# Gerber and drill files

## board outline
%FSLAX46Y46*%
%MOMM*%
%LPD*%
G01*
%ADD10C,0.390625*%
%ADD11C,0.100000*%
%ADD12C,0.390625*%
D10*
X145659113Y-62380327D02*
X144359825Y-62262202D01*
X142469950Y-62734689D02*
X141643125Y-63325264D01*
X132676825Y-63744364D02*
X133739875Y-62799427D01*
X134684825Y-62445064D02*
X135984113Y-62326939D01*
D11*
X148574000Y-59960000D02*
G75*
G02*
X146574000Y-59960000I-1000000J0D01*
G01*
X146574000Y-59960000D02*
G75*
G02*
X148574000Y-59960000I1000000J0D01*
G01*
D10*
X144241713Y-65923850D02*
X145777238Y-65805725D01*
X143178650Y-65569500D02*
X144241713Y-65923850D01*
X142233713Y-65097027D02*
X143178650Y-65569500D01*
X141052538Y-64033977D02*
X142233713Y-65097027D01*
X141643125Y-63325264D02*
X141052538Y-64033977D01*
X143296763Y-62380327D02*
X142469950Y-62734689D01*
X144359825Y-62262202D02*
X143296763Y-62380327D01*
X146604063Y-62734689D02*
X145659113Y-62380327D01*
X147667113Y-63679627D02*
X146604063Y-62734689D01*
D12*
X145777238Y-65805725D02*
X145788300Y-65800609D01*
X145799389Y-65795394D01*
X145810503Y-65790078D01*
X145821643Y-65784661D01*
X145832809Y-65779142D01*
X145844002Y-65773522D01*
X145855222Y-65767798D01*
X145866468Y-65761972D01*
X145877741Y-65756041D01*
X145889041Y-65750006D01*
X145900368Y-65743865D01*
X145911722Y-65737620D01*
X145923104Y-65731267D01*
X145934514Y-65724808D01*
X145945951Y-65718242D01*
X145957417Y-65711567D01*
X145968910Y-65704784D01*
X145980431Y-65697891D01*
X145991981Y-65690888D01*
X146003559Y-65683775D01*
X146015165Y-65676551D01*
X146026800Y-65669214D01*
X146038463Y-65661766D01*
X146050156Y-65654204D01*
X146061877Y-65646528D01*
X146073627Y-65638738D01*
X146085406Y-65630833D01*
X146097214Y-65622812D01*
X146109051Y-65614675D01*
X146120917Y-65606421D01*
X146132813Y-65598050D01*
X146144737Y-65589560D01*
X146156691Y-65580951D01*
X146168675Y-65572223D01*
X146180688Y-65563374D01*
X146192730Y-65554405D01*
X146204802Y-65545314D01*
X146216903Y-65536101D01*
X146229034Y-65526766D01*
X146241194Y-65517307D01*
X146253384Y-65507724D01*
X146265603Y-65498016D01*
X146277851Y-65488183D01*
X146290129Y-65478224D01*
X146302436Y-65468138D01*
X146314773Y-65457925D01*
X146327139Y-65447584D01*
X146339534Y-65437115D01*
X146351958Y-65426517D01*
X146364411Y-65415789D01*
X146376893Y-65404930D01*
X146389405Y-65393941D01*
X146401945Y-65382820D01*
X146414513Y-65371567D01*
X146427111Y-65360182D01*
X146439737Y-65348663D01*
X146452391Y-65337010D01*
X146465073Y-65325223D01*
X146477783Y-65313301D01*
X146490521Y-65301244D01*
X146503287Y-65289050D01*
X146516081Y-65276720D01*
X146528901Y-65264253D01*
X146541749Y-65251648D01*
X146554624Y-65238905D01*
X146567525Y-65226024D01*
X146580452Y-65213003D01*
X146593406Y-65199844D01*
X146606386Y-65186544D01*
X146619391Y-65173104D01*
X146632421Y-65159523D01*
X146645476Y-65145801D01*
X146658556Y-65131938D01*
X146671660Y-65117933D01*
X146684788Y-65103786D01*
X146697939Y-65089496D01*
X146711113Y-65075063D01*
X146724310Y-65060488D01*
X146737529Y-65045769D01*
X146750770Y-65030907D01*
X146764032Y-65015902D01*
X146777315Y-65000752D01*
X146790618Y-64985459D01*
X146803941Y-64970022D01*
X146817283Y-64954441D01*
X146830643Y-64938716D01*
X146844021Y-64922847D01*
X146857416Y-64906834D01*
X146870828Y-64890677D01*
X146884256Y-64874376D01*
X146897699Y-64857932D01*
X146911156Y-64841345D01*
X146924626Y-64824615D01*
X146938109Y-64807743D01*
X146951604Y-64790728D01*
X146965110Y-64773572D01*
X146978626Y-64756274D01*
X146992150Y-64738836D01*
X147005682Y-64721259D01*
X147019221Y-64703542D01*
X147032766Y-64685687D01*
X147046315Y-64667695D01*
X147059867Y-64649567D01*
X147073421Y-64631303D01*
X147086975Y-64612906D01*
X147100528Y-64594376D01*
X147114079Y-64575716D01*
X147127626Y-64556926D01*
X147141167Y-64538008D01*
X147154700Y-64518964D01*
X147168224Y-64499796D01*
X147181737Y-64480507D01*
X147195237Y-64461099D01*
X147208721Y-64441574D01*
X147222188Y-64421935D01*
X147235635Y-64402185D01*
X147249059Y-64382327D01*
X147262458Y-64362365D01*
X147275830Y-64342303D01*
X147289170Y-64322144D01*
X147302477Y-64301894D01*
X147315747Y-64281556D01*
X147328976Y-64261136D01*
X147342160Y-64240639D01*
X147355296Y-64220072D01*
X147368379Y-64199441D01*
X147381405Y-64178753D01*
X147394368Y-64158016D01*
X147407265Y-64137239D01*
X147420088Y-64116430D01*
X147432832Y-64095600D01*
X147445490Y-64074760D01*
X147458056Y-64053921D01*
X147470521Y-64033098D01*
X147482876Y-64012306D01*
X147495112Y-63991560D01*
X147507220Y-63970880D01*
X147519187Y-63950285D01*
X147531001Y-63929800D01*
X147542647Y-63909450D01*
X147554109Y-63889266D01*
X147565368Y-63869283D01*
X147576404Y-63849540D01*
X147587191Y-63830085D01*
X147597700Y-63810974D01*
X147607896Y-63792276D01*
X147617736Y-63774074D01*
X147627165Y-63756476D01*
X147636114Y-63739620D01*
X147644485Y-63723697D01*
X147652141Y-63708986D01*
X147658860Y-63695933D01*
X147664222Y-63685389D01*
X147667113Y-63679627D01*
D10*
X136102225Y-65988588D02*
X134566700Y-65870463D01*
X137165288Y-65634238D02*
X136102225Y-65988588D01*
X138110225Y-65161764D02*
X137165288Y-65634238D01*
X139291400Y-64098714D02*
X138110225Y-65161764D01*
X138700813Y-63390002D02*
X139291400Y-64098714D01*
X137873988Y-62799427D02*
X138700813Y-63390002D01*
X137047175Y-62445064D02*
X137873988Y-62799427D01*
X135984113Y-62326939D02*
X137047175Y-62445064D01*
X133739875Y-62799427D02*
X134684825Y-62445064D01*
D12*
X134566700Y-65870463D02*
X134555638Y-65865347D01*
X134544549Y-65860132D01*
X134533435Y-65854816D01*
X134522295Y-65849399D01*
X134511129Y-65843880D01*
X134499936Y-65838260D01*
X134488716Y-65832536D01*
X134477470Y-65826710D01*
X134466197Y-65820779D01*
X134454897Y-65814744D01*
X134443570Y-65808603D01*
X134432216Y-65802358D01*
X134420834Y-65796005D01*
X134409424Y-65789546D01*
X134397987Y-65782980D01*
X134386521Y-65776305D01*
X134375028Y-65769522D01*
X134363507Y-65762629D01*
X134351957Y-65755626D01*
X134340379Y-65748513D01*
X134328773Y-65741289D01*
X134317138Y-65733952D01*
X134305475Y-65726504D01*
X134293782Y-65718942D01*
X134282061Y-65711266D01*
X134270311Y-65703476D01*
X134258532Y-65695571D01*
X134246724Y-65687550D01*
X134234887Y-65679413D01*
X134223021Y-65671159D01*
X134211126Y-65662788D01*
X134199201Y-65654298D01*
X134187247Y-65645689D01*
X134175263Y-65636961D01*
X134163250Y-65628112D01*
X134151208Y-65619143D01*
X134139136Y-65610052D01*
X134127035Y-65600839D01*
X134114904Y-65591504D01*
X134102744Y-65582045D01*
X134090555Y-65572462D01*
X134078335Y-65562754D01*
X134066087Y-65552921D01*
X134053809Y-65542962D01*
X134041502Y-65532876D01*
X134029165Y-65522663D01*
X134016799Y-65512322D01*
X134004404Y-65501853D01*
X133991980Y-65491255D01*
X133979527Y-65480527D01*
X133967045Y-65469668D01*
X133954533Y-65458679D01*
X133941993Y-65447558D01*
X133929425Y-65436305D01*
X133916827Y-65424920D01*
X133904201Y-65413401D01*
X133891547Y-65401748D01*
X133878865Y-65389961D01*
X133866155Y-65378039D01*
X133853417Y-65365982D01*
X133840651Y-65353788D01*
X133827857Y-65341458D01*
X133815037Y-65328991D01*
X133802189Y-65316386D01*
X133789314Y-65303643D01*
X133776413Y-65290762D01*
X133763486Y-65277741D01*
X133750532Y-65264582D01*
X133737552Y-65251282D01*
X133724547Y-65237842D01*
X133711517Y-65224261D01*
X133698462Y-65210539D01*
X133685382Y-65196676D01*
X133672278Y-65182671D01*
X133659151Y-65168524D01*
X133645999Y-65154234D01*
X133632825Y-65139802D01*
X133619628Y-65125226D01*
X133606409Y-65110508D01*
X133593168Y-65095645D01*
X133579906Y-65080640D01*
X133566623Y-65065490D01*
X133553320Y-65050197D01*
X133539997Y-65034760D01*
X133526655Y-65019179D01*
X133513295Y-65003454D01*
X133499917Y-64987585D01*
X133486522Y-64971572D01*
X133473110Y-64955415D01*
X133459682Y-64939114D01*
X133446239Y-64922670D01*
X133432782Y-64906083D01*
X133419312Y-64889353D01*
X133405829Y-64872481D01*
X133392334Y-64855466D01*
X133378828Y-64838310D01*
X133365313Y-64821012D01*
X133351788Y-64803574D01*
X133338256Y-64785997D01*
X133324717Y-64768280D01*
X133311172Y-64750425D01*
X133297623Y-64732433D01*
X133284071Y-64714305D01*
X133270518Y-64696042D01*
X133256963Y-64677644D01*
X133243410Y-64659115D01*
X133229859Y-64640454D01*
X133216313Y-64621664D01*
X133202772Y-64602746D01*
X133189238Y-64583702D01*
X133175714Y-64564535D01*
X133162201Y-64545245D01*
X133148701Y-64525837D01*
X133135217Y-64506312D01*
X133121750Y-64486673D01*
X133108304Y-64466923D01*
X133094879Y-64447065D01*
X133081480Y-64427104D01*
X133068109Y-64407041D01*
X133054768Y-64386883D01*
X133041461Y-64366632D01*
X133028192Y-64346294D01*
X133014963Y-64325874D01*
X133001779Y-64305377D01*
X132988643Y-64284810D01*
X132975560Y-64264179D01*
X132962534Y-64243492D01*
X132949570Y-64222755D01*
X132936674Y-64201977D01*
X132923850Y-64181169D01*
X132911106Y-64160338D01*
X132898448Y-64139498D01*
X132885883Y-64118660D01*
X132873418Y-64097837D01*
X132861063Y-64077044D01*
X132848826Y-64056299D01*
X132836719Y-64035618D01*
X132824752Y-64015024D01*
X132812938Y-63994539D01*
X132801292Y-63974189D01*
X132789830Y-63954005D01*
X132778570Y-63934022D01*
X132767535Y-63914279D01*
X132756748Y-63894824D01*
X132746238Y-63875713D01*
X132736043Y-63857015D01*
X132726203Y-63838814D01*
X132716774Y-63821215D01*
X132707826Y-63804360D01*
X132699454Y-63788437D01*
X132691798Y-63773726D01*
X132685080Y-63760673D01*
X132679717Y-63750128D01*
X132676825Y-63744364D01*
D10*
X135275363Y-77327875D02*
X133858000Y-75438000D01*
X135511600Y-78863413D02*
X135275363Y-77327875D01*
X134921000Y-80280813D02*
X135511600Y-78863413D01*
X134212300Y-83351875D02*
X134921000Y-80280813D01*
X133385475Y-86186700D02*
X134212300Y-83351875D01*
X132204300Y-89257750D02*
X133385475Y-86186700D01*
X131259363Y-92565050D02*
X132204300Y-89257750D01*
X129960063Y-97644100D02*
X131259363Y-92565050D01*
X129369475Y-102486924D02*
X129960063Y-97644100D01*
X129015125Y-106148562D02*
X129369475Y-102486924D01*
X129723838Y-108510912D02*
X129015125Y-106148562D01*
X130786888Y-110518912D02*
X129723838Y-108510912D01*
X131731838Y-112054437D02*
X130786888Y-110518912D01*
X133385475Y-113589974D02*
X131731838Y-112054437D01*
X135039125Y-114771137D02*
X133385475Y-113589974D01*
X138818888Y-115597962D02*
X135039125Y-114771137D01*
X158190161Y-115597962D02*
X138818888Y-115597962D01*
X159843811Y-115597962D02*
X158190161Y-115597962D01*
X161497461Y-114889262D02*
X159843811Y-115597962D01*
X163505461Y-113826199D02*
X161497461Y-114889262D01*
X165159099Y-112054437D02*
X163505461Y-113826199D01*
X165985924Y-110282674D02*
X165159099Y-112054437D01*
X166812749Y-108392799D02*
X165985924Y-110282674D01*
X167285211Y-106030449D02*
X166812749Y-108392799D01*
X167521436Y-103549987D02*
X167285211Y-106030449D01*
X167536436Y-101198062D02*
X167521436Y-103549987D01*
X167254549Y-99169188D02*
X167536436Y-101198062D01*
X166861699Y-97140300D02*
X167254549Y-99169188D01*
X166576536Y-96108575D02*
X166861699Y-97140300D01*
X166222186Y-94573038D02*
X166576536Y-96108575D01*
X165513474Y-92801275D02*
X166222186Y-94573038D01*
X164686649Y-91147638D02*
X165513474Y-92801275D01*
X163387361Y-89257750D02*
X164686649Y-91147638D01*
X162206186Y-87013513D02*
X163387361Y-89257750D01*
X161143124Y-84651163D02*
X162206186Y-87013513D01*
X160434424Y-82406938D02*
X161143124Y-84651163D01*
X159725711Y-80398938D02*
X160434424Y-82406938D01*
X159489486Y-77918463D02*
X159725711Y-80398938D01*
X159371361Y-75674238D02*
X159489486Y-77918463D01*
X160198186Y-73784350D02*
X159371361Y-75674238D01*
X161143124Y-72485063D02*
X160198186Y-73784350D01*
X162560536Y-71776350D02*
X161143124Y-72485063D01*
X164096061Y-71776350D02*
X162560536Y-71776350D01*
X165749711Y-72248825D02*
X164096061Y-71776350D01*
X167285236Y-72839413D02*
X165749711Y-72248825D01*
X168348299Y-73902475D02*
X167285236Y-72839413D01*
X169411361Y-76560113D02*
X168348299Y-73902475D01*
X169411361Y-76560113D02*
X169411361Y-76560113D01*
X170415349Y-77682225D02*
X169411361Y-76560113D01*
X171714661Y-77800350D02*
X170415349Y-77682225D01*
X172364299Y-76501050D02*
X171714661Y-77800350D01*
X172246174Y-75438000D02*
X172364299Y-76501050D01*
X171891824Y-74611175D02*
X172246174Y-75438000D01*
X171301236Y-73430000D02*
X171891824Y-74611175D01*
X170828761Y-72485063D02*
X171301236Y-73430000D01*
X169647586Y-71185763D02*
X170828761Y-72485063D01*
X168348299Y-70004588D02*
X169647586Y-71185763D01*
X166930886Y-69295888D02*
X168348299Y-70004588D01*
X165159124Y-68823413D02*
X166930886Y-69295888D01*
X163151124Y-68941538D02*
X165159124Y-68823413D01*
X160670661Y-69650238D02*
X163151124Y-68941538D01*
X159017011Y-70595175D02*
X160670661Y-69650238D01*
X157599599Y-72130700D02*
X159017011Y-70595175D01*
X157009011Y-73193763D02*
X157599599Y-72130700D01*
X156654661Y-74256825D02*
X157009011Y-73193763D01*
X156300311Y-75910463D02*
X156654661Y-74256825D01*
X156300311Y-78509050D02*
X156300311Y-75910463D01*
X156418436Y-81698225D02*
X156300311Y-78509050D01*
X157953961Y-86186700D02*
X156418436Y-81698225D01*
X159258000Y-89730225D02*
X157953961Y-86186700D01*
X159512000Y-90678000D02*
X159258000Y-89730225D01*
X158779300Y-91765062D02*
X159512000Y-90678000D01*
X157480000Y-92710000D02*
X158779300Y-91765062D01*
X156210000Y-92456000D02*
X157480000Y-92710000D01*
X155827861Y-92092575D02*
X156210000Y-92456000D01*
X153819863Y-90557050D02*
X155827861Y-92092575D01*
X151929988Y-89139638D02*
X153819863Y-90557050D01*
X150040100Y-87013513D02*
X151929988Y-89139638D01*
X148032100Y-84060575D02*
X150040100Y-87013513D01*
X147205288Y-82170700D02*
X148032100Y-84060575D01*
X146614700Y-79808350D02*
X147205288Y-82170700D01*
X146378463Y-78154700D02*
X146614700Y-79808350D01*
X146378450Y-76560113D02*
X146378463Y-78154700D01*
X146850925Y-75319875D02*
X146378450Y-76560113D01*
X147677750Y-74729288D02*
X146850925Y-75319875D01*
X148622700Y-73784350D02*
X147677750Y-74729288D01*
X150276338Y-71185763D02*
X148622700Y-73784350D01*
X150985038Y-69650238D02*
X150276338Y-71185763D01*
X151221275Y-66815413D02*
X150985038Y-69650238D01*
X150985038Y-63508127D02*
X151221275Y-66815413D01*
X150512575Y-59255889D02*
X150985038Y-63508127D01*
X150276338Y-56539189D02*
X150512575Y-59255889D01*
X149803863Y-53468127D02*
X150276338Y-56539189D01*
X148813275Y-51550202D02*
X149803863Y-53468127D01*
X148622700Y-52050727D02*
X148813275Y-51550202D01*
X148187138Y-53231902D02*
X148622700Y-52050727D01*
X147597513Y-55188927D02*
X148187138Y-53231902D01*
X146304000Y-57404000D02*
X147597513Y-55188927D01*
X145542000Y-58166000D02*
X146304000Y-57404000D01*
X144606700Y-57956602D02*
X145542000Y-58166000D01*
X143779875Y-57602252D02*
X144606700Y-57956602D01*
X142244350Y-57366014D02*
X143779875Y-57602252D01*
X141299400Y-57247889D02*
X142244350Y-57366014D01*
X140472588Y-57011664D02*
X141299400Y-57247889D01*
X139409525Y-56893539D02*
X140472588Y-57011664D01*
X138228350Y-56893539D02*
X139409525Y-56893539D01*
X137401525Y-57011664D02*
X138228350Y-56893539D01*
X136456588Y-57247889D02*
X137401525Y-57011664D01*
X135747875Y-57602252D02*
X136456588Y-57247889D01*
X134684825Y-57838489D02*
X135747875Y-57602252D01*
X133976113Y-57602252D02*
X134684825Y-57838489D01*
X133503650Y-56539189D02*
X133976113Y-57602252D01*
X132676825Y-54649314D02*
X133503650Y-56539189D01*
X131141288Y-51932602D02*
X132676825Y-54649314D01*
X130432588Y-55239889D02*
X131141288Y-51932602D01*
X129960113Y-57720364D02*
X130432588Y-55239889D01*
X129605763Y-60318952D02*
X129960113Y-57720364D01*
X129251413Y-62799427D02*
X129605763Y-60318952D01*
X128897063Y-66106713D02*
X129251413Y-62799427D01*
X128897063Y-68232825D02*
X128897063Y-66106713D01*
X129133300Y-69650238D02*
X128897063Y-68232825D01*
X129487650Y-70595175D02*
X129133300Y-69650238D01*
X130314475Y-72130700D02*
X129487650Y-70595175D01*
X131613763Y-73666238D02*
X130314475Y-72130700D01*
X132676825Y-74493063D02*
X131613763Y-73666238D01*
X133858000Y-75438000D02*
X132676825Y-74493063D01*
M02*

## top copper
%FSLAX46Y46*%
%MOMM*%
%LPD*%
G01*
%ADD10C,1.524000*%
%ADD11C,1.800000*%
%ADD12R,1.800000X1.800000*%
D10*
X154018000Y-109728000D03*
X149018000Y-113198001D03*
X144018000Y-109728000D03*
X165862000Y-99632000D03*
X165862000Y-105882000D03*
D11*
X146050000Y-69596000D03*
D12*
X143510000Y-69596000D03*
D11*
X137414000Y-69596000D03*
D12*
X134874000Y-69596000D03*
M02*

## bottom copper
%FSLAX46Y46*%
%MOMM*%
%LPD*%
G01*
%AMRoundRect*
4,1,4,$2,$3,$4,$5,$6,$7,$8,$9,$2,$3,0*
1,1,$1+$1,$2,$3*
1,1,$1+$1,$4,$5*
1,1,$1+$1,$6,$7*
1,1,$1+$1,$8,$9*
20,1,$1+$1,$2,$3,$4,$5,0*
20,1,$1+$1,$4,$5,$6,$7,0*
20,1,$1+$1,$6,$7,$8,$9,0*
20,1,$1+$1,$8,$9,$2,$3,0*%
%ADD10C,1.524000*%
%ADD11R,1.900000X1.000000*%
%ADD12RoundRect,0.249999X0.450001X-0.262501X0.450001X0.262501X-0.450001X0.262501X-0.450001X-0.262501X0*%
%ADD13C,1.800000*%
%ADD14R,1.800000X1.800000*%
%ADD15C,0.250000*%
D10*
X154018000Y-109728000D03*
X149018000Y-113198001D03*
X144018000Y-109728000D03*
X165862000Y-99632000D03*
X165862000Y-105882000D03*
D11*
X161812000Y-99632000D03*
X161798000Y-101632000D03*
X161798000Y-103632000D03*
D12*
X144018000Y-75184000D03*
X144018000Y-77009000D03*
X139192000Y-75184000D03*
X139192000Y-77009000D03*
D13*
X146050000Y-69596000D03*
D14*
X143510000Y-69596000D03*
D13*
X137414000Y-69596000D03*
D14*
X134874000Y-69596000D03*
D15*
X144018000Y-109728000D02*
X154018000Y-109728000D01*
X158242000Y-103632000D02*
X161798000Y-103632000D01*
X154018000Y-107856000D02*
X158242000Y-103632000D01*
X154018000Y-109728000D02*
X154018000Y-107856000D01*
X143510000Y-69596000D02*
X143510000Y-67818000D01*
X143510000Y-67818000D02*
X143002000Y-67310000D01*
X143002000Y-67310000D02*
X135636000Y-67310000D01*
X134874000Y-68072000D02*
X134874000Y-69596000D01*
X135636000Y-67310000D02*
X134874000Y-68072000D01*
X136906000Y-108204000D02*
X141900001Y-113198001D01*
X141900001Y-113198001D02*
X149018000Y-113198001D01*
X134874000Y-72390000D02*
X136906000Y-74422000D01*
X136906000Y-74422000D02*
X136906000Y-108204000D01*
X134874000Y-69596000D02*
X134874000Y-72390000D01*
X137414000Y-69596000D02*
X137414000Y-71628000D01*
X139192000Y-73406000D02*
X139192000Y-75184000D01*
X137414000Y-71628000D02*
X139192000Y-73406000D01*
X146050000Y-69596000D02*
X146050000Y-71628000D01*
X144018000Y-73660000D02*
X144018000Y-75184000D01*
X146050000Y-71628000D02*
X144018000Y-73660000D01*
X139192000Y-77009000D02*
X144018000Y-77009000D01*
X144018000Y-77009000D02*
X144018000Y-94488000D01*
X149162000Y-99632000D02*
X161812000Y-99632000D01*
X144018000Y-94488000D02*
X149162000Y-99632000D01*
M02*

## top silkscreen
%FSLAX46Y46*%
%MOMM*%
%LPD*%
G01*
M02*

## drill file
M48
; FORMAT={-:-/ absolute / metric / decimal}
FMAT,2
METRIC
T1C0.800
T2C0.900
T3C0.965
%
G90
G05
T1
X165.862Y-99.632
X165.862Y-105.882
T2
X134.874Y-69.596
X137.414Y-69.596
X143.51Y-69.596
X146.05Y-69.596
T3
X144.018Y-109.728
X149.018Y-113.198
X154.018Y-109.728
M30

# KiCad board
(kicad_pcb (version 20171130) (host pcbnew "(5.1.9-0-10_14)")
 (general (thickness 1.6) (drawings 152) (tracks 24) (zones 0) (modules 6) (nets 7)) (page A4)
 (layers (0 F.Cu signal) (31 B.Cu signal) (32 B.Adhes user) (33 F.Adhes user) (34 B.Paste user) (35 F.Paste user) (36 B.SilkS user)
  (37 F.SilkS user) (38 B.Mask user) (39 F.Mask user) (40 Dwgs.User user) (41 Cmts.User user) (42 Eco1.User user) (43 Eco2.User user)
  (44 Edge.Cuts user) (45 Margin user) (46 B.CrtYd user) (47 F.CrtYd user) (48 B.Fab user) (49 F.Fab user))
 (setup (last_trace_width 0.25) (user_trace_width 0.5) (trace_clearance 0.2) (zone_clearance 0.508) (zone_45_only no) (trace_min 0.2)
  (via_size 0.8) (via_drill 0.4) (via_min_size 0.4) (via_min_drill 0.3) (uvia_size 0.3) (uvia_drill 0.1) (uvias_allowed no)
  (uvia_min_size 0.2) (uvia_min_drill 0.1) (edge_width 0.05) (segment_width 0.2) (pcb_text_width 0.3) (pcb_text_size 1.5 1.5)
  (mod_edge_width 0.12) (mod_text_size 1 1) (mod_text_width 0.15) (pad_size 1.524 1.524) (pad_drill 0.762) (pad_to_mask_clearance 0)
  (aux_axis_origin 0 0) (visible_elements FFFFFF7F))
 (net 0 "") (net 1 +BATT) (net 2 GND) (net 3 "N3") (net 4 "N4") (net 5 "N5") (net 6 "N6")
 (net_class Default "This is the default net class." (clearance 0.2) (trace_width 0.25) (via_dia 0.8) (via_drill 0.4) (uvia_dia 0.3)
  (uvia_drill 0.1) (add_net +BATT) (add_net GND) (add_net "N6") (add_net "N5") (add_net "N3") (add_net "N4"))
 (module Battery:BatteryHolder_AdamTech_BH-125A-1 (layer B.Cu) (at 144.018 109.728)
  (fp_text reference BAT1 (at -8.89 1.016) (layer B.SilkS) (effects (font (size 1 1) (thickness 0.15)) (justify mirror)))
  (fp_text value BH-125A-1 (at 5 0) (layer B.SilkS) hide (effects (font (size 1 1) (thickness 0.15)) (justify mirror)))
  (pad POS2 thru_hole circle (at 10 0) (size 1.524 1.524) (drill 0.9652) (layers *.Cu *.Mask) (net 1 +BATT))
  (pad NEG thru_hole circle (at 5 3.470001) (size 1.524 1.524) (drill 0.9652) (layers *.Cu *.Mask) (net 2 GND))
  (pad POS1 thru_hole circle (at 0 0) (size 1.524 1.524) (drill 0.9652) (layers *.Cu *.Mask) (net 1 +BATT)))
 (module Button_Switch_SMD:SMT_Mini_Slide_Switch (layer B.Cu) (at 163.576 102.757 270)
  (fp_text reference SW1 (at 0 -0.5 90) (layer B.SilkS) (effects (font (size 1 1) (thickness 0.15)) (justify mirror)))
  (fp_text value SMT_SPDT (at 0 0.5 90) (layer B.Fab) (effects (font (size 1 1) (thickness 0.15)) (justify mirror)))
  (pad "" thru_hole circle (at -3.125 -2.286 270) (size 1.524 1.524) (drill 0.8) (layers *.Cu *.Mask))
  (pad "" thru_hole circle (at 3.125 -2.286 270) (size 1.524 1.524) (drill 0.8) (layers *.Cu *.Mask))
  (pad 1 smd rect (at -3.125 1.764 270) (size 1 1.9) (layers B.Cu B.Paste B.Mask) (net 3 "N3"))
  (pad 2 smd rect (at -1.125 1.778 270) (size 1 1.9) (layers B.Cu B.Paste B.Mask) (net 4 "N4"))
  (pad 3 smd rect (at 0.875 1.778 270) (size 1 1.9) (layers B.Cu B.Paste B.Mask) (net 1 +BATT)))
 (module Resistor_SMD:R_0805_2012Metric (layer B.Cu) (at 144.018 76.0965 90)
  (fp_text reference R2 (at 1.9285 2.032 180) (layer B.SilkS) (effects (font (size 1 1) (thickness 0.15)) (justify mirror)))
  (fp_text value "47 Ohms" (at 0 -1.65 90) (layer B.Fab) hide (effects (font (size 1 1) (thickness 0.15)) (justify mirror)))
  (pad 2 smd roundrect (at 0.9125 0 90) (size 1.025 1.4) (layers B.Cu B.Paste B.Mask) (roundrect_rratio 0.2439014634146341) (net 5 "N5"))
  (pad 1 smd roundrect (at -0.9125 0 90) (size 1.025 1.4) (layers B.Cu B.Paste B.Mask) (roundrect_rratio 0.2439014634146341) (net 3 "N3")))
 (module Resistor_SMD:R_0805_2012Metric (layer B.Cu) (at 139.192 76.0965 90)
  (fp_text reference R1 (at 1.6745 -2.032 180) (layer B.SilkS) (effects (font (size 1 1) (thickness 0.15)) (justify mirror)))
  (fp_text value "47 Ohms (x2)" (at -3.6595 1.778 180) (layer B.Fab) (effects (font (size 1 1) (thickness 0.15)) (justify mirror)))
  (pad 2 smd roundrect (at 0.9125 0 90) (size 1.025 1.4) (layers B.Cu B.Paste B.Mask) (roundrect_rratio 0.2439014634146341) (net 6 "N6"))
  (pad 1 smd roundrect (at -0.9125 0 90) (size 1.025 1.4) (layers B.Cu B.Paste B.Mask) (roundrect_rratio 0.2439014634146341) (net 3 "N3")))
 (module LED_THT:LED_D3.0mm (layer B.Cu) (at 143.51 69.596)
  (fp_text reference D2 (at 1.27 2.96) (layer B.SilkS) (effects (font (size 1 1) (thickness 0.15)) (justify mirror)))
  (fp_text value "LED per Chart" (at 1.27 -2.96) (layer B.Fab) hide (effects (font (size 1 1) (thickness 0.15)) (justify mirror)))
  (pad 2 thru_hole circle (at 2.54 0) (size 1.8 1.8) (drill 0.9) (layers *.Cu *.Mask) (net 5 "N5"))
  (pad 1 thru_hole rect (at 0 0) (size 1.8 1.8) (drill 0.9) (layers *.Cu *.Mask) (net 2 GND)))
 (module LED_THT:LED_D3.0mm (layer B.Cu) (at 134.874 69.596)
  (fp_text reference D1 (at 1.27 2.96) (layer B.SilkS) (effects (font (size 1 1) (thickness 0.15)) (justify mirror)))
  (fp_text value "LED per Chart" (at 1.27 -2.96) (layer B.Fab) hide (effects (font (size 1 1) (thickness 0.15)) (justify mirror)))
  (pad 2 thru_hole circle (at 2.54 0) (size 1.8 1.8) (drill 0.9) (layers *.Cu *.Mask) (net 6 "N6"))
  (pad 1 thru_hole rect (at 0 0) (size 1.8 1.8) (drill 0.9) (layers *.Cu *.Mask) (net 2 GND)))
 (gr_line (start 145.659113 62.380327) (end 144.359825 62.262202) (layer Edge.Cuts) (width 0.390625))
 (gr_line (start 142.46995 62.734689) (end 141.643125 63.325264) (layer Edge.Cuts) (width 0.390625))
 (gr_line (start 132.676825 63.744364) (end 133.739875 62.799427) (layer Edge.Cuts) (width 0.390625))
 (gr_line (start 134.684825 62.445064) (end 135.984113 62.326939) (layer Edge.Cuts) (width 0.390625))
 (gr_circle (center 147.574 59.96) (end 148.574 59.96) (layer Edge.Cuts) (width 0.1))
 (gr_line (start 144.241713 65.92385) (end 145.777238 65.805725) (layer Edge.Cuts) (width 0.390625))
 (gr_line (start 143.17865 65.5695) (end 144.241713 65.92385) (layer Edge.Cuts) (width 0.390625))
 (gr_line (start 142.233713 65.097027) (end 143.17865 65.5695) (layer Edge.Cuts) (width 0.390625))
 (gr_line (start 141.052538 64.033977) (end 142.233713 65.097027) (layer Edge.Cuts) (width 0.390625))
 (gr_line (start 141.643125 63.325264) (end 141.052538 64.033977) (layer Edge.Cuts) (width 0.390625))
 (gr_line (start 143.296763 62.380327) (end 142.46995 62.734689) (layer Edge.Cuts) (width 0.390625))
 (gr_line (start 144.359825 62.262202) (end 143.296763 62.380327) (layer Edge.Cuts) (width 0.390625))
 (gr_line (start 146.604063 62.734689) (end 145.659113 62.380327) (layer Edge.Cuts) (width 0.390625))
 (gr_line (start 147.667113 63.679627) (end 146.604063 62.734689) (layer Edge.Cuts) (width 0.390625))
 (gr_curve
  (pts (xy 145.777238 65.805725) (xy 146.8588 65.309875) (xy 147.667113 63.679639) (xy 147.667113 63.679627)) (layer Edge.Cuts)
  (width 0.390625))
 (gr_line (start 136.102225 65.988588) (end 134.5667 65.870463) (layer Edge.Cuts) (width 0.390625))
 (gr_line (start 137.165288 65.634238) (end 136.102225 65.988588) (layer Edge.Cuts) (width 0.390625))
 (gr_line (start 138.110225 65.161764) (end 137.165288 65.634238) (layer Edge.Cuts) (width 0.390625))
 (gr_line (start 139.2914 64.098714) (end 138.110225 65.161764) (layer Edge.Cuts) (width 0.390625))
 (gr_line (start 138.700813 63.390002) (end 139.2914 64.098714) (layer Edge.Cuts) (width 0.390625))
 (gr_line (start 137.873988 62.799427) (end 138.700813 63.390002) (layer Edge.Cuts) (width 0.390625))
 (gr_line (start 137.047175 62.445064) (end 137.873988 62.799427) (layer Edge.Cuts) (width 0.390625))
 (gr_line (start 135.984113 62.326939) (end 137.047175 62.445064) (layer Edge.Cuts) (width 0.390625))
 (gr_line (start 133.739875 62.799427) (end 134.684825 62.445064) (layer Edge.Cuts) (width 0.390625))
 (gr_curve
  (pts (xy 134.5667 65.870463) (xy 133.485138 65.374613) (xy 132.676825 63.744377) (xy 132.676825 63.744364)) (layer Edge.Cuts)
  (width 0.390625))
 (gr_line (start 135.275363 77.327875) (end 133.858 75.438) (layer Edge.Cuts) (width 0.390625))
 (gr_line (start 135.5116 78.863413) (end 135.275363 77.327875) (layer Edge.Cuts) (width 0.390625))
 (gr_line (start 134.921 80.280813) (end 135.5116 78.863413) (layer Edge.Cuts) (width 0.390625))
 (gr_line (start 134.2123 83.351875) (end 134.921 80.280813) (layer Edge.Cuts) (width 0.390625))
 (gr_line (start 133.385475 86.1867) (end 134.2123 83.351875) (layer Edge.Cuts) (width 0.390625))
 (gr_line (start 132.2043 89.25775) (end 133.385475 86.1867) (layer Edge.Cuts) (width 0.390625))
 (gr_line (start 131.259363 92.56505) (end 132.2043 89.25775) (layer Edge.Cuts) (width 0.390625))
 (gr_line (start 129.960063 97.6441) (end 131.259363 92.56505) (layer Edge.Cuts) (width 0.390625))
 (gr_line (start 129.369475 102.486924) (end 129.960063 97.6441) (layer Edge.Cuts) (width 0.390625))
 (gr_line (start 129.015125 106.148562) (end 129.369475 102.486924) (layer Edge.Cuts) (width 0.390625))
 (gr_line (start 129.723838 108.510912) (end 129.015125 106.148562) (layer Edge.Cuts) (width 0.390625))
 (gr_line (start 130.786888 110.518912) (end 129.723838 108.510912) (layer Edge.Cuts) (width 0.390625))
 (gr_line (start 131.731838 112.054437) (end 130.786888 110.518912) (layer Edge.Cuts) (width 0.390625))
 (gr_line (start 133.385475 113.589974) (end 131.731838 112.054437) (layer Edge.Cuts) (width 0.390625))
 (gr_line (start 135.039125 114.771137) (end 133.385475 113.589974) (layer Edge.Cuts) (width 0.390625))
 (gr_line (start 138.818888 115.597962) (end 135.039125 114.771137) (layer Edge.Cuts) (width 0.390625))
 (gr_line (start 158.190161 115.597962) (end 138.818888 115.597962) (layer Edge.Cuts) (width 0.390625))
 (gr_line (start 159.843811 115.597962) (end 158.190161 115.597962) (layer Edge.Cuts) (width 0.390625))
 (gr_line (start 161.497461 114.889262) (end 159.843811 115.597962) (layer Edge.Cuts) (width 0.390625))
 (gr_line (start 163.505461 113.826199) (end 161.497461 114.889262) (layer Edge.Cuts) (width 0.390625))
 (gr_line (start 165.159099 112.054437) (end 163.505461 113.826199) (layer Edge.Cuts) (width 0.390625))
 (gr_line (start 165.985924 110.282674) (end 165.159099 112.054437) (layer Edge.Cuts) (width 0.390625))
 (gr_line (start 166.812749 108.392799) (end 165.985924 110.282674) (layer Edge.Cuts) (width 0.390625))
 (gr_line (start 167.285211 106.030449) (end 166.812749 108.392799) (layer Edge.Cuts) (width 0.390625))
 (gr_line (start 167.521436 103.549987) (end 167.285211 106.030449) (layer Edge.Cuts) (width 0.390625))
 (gr_line (start 167.536436 101.198062) (end 167.521436 103.549987) (layer Edge.Cuts) (width 0.390625))
 (gr_line (start 167.254549 99.169188) (end 167.536436 101.198062) (layer Edge.Cuts) (width 0.390625))
 (gr_line (start 166.861699 97.1403) (end 167.254549 99.169188) (layer Edge.Cuts) (width 0.390625))
 (gr_line (start 166.576536 96.108575) (end 166.861699 97.1403) (layer Edge.Cuts) (width 0.390625))
 (gr_line (start 166.222186 94.573038) (end 166.576536 96.108575) (layer Edge.Cuts) (width 0.390625))
 (gr_line (start 165.513474 92.801275) (end 166.222186 94.573038) (layer Edge.Cuts) (width 0.390625))
 (gr_line (start 164.686649 91.147638) (end 165.513474 92.801275) (layer Edge.Cuts) (width 0.390625))
 (gr_line (start 163.387361 89.25775) (end 164.686649 91.147638) (layer Edge.Cuts) (width 0.390625))
 (gr_line (start 162.206186 87.013513) (end 163.387361 89.25775) (layer Edge.Cuts) (width 0.390625))
 (gr_line (start 161.143124 84.651163) (end 162.206186 87.013513) (layer Edge.Cuts) (width 0.390625))
 (gr_line (start 160.434424 82.406938) (end 161.143124 84.651163) (layer Edge.Cuts) (width 0.390625))
 (gr_line (start 159.725711 80.398938) (end 160.434424 82.406938) (layer Edge.Cuts) (width 0.390625))
 (gr_line (start 159.489486 77.918463) (end 159.725711 80.398938) (layer Edge.Cuts) (width 0.390625))
 (gr_line (start 159.371361 75.674238) (end 159.489486 77.918463) (layer Edge.Cuts) (width 0.390625))
 (gr_line (start 160.198186 73.78435) (end 159.371361 75.674238) (layer Edge.Cuts) (width 0.390625))
 (gr_line (start 161.143124 72.485063) (end 160.198186 73.78435) (layer Edge.Cuts) (width 0.390625))
 (gr_line (start 162.560536 71.77635) (end 161.143124 72.485063) (layer Edge.Cuts) (width 0.390625))
 (gr_line (start 164.096061 71.77635) (end 162.560536 71.77635) (layer Edge.Cuts) (width 0.390625))
 (gr_line (start 165.749711 72.248825) (end 164.096061 71.77635) (layer Edge.Cuts) (width 0.390625))
 (gr_line (start 167.285236 72.839413) (end 165.749711 72.248825) (layer Edge.Cuts) (width 0.390625))
 (gr_line (start 168.348299 73.902475) (end 167.285236 72.839413) (layer Edge.Cuts) (width 0.390625))
 (gr_line (start 169.411361 76.560113) (end 168.348299 73.902475) (layer Edge.Cuts) (width 0.390625))
 (gr_line (start 169.411361 76.560113) (end 169.411361 76.560113) (layer Edge.Cuts) (width 0.390625))
 (gr_line (start 170.415349 77.682225) (end 169.411361 76.560113) (layer Edge.Cuts) (width 0.390625))
 (gr_line (start 171.714661 77.80035) (end 170.415349 77.682225) (layer Edge.Cuts) (width 0.390625))
 (gr_line (start 172.364299 76.50105) (end 171.714661 77.80035) (layer Edge.Cuts) (width 0.390625))
 (gr_line (start 172.246174 75.438) (end 172.364299 76.50105) (layer Edge.Cuts) (width 0.390625))
 (gr_line (start 171.891824 74.611175) (end 172.246174 75.438) (layer Edge.Cuts) (width 0.390625))
 (gr_line (start 171.301236 73.43) (end 171.891824 74.611175) (layer Edge.Cuts) (width 0.390625))
 (gr_line (start 170.828761 72.485063) (end 171.301236 73.43) (layer Edge.Cuts) (width 0.390625))
 (gr_line (start 169.647586 71.185763) (end 170.828761 72.485063) (layer Edge.Cuts) (width 0.390625))
 (gr_line (start 168.348299 70.004588) (end 169.647586 71.185763) (layer Edge.Cuts) (width 0.390625))
 (gr_line (start 166.930886 69.295888) (end 168.348299 70.004588) (layer Edge.Cuts) (width 0.390625))
 (gr_line (start 165.159124 68.823413) (end 166.930886 69.295888) (layer Edge.Cuts) (width 0.390625))
 (gr_line (start 163.151124 68.941538) (end 165.159124 68.823413) (layer Edge.Cuts) (width 0.390625))
 (gr_line (start 160.670661 69.650238) (end 163.151124 68.941538) (layer Edge.Cuts) (width 0.390625))
 (gr_line (start 159.017011 70.595175) (end 160.670661 69.650238) (layer Edge.Cuts) (width 0.390625))
 (gr_line (start 157.599599 72.1307) (end 159.017011 70.595175) (layer Edge.Cuts) (width 0.390625))
 (gr_line (start 157.009011 73.193763) (end 157.599599 72.1307) (layer Edge.Cuts) (width 0.390625))
 (gr_line (start 156.654661 74.256825) (end 157.009011 73.193763) (layer Edge.Cuts) (width 0.390625))
 (gr_line (start 156.300311 75.910463) (end 156.654661 74.256825) (layer Edge.Cuts) (width 0.390625))
 (gr_line (start 156.300311 78.50905) (end 156.300311 75.910463) (layer Edge.Cuts) (width 0.390625))
 (gr_line (start 156.418436 81.698225) (end 156.300311 78.50905) (layer Edge.Cuts) (width 0.390625))
 (gr_line (start 157.953961 86.1867) (end 156.418436 81.698225) (layer Edge.Cuts) (width 0.390625))
 (gr_line (start 159.258 89.730225) (end 157.953961 86.1867) (layer Edge.Cuts) (width 0.390625))
 (gr_line (start 159.512 90.678) (end 159.258 89.730225) (layer Edge.Cuts) (width 0.390625))
 (gr_line (start 158.7793 91.765062) (end 159.512 90.678) (layer Edge.Cuts) (width 0.390625))
 (gr_line (start 157.48 92.71) (end 158.7793 91.765062) (layer Edge.Cuts) (width 0.390625))
 (gr_line (start 156.21 92.456) (end 157.48 92.71) (layer Edge.Cuts) (width 0.390625))
 (gr_line (start 155.827861 92.092575) (end 156.21 92.456) (layer Edge.Cuts) (width 0.390625))
 (gr_line (start 153.819863 90.55705) (end 155.827861 92.092575) (layer Edge.Cuts) (width 0.390625))
 (gr_line (start 151.929988 89.139638) (end 153.819863 90.55705) (layer Edge.Cuts) (width 0.390625))
 (gr_line (start 150.0401 87.013513) (end 151.929988 89.139638) (layer Edge.Cuts) (width 0.390625))
 (gr_line (start 148.0321 84.060575) (end 150.0401 87.013513) (layer Edge.Cuts) (width 0.390625))
 (gr_line (start 147.205288 82.1707) (end 148.0321 84.060575) (layer Edge.Cuts) (width 0.390625))
 (gr_line (start 146.6147 79.80835) (end 147.205288 82.1707) (layer Edge.Cuts) (width 0.390625))
 (gr_line (start 146.378463 78.1547) (end 146.6147 79.80835) (layer Edge.Cuts) (width 0.390625))
 (gr_line (start 146.37845 76.560113) (end 146.378463 78.1547) (layer Edge.Cuts) (width 0.390625))
 (gr_line (start 146.850925 75.319875) (end 146.37845 76.560113) (layer Edge.Cuts) (width 0.390625))
 (gr_line (start 147.67775 74.729288) (end 146.850925 75.319875) (layer Edge.Cuts) (width 0.390625))
 (gr_line (start 148.6227 73.78435) (end 147.67775 74.729288) (layer Edge.Cuts) (width 0.390625))
 (gr_line (start 150.276338 71.185763) (end 148.6227 73.78435) (layer Edge.Cuts) (width 0.390625))
 (gr_line (start 150.985038 69.650238) (end 150.276338 71.185763) (layer Edge.Cuts) (width 0.390625))
 (gr_line (start 151.221275 66.815413) (end 150.985038 69.650238) (layer Edge.Cuts) (width 0.390625))
 (gr_line (start 150.985038 63.508127) (end 151.221275 66.815413) (layer Edge.Cuts) (width 0.390625))
 (gr_line (start 150.512575 59.255889) (end 150.985038 63.508127) (layer Edge.Cuts) (width 0.390625))
 (gr_line (start 150.276338 56.539189) (end 150.512575 59.255889) (layer Edge.Cuts) (width 0.390625))
 (gr_line (start 149.803863 53.468127) (end 150.276338 56.539189) (layer Edge.Cuts) (width 0.390625))
 (gr_line (start 148.813275 51.550202) (end 149.803863 53.468127) (layer Edge.Cuts) (width 0.390625))
 (gr_line (start 148.6227 52.050727) (end 148.813275 51.550202) (layer Edge.Cuts) (width 0.390625))
 (gr_line (start 148.187138 53.231902) (end 148.6227 52.050727) (layer Edge.Cuts) (width 0.390625))
 (gr_line (start 147.597513 55.188927) (end 148.187138 53.231902) (layer Edge.Cuts) (width 0.390625))
 (gr_line (start 146.304 57.404) (end 147.597513 55.188927) (layer Edge.Cuts) (width 0.390625))
 (gr_line (start 145.542 58.166) (end 146.304 57.404) (layer Edge.Cuts) (width 0.390625))
 (gr_line (start 144.6067 57.956602) (end 145.542 58.166) (layer Edge.Cuts) (width 0.390625))
 (gr_line (start 143.779875 57.602252) (end 144.6067 57.956602) (layer Edge.Cuts) (width 0.390625))
 (gr_line (start 142.24435 57.366014) (end 143.779875 57.602252) (layer Edge.Cuts) (width 0.390625))
 (gr_line (start 141.2994 57.247889) (end 142.24435 57.366014) (layer Edge.Cuts) (width 0.390625))
 (gr_line (start 140.472588 57.011664) (end 141.2994 57.247889) (layer Edge.Cuts) (width 0.390625))
 (gr_line (start 139.409525 56.893539) (end 140.472588 57.011664) (layer Edge.Cuts) (width 0.390625))
 (gr_line (start 138.22835 56.893539) (end 139.409525 56.893539) (layer Edge.Cuts) (width 0.390625))
 (gr_line (start 137.401525 57.011664) (end 138.22835 56.893539) (layer Edge.Cuts) (width 0.390625))
 (gr_line (start 136.456588 57.247889) (end 137.401525 57.011664) (layer Edge.Cuts) (width 0.390625))
 (gr_line (start 135.747875 57.602252) (end 136.456588 57.247889) (layer Edge.Cuts) (width 0.390625))
 (gr_line (start 134.684825 57.838489) (end 135.747875 57.602252) (layer Edge.Cuts) (width 0.390625))
 (gr_line (start 133.976113 57.602252) (end 134.684825 57.838489) (layer Edge.Cuts) (width 0.390625))
 (gr_line (start 133.50365 56.539189) (end 133.976113 57.602252) (layer Edge.Cuts) (width 0.390625))
 (gr_line (start 132.676825 54.649314) (end 133.50365 56.539189) (layer Edge.Cuts) (width 0.390625))
 (gr_line (start 131.141288 51.932602) (end 132.676825 54.649314) (layer Edge.Cuts) (width 0.390625))
 (gr_line (start 130.432588 55.239889) (end 131.141288 51.932602) (layer Edge.Cuts) (width 0.390625))
 (gr_line (start 129.960113 57.720364) (end 130.432588 55.239889) (layer Edge.Cuts) (width 0.390625))
 (gr_line (start 129.605763 60.318952) (end 129.960113 57.720364) (layer Edge.Cuts) (width 0.390625))
 (gr_line (start 129.251413 62.799427) (end 129.605763 60.318952) (layer Edge.Cuts) (width 0.390625))
 (gr_line (start 128.897063 66.106713) (end 129.251413 62.799427) (layer Edge.Cuts) (width 0.390625))
 (gr_line (start 128.897063 68.232825) (end 128.897063 66.106713) (layer Edge.Cuts) (width 0.390625))
 (gr_line (start 129.1333 69.650238) (end 128.897063 68.232825) (layer Edge.Cuts) (width 0.390625))
 (gr_line (start 129.48765 70.595175) (end 129.1333 69.650238) (layer Edge.Cuts) (width 0.390625))
 (gr_line (start 130.314475 72.1307) (end 129.48765 70.595175) (layer Edge.Cuts) (width 0.390625))
 (gr_line (start 131.613763 73.666238) (end 130.314475 72.1307) (layer Edge.Cuts) (width 0.390625))
 (gr_line (start 132.676825 74.493063) (end 131.613763 73.666238) (layer Edge.Cuts) (width 0.390625))
 (gr_line (start 133.858 75.438) (end 132.676825 74.493063) (layer Edge.Cuts) (width 0.390625))
 (segment (start 144.018 109.728) (end 154.018 109.728) (width 0.25) (layer B.Cu) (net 1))
 (segment (start 158.242 103.632) (end 161.798 103.632) (width 0.25) (layer B.Cu) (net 1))
 (segment (start 154.018 107.856) (end 158.242 103.632) (width 0.25) (layer B.Cu) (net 1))
 (segment (start 154.018 109.728) (end 154.018 107.856) (width 0.25) (layer B.Cu) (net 1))
 (segment (start 143.51 69.596) (end 143.51 67.818) (width 0.25) (layer B.Cu) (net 2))
 (segment (start 143.51 67.818) (end 143.002 67.31) (width 0.25) (layer B.Cu) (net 2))
 (segment (start 143.002 67.31) (end 135.636 67.31) (width 0.25) (layer B.Cu) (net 2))
 (segment (start 134.874 68.072) (end 134.874 69.596) (width 0.25) (layer B.Cu) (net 2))
 (segment (start 135.636 67.31) (end 134.874 68.072) (width 0.25) (layer B.Cu) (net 2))
 (segment (start 136.906 108.204) (end 141.900001 113.198001) (width 0.25) (layer B.Cu) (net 2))
 (segment (start 141.900001 113.198001) (end 149.018 113.198001) (width 0.25) (layer B.Cu) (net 2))
 (segment (start 134.874 72.39) (end 136.906 74.422) (width 0.25) (layer B.Cu) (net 2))
 (segment (start 136.906 74.422) (end 136.906 108.204) (width 0.25) (layer B.Cu) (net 2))
 (segment (start 134.874 69.596) (end 134.874 72.39) (width 0.25) (layer B.Cu) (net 2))
 (segment (start 137.414 69.596) (end 137.414 71.628) (width 0.25) (layer B.Cu) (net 6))
 (segment (start 139.192 73.406) (end 139.192 75.184) (width 0.25) (layer B.Cu) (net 6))
 (segment (start 137.414 71.628) (end 139.192 73.406) (width 0.25) (layer B.Cu) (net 6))
 (segment (start 146.05 69.596) (end 146.05 71.628) (width 0.25) (layer B.Cu) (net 5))
 (segment (start 144.018 73.66) (end 144.018 75.184) (width 0.25) (layer B.Cu) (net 5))
 (segment (start 146.05 71.628) (end 144.018 73.66) (width 0.25) (layer B.Cu) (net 5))
 (segment (start 139.192 77.009) (end 144.018 77.009) (width 0.25) (layer B.Cu) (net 3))
 (segment (start 144.018 77.009) (end 144.018 94.488) (width 0.25) (layer B.Cu) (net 3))
 (segment (start 149.162 99.632) (end 161.812 99.632) (width 0.25) (layer B.Cu) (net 3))
 (segment (start 144.018 94.488) (end 149.162 99.632) (width 0.25) (layer B.Cu) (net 3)))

